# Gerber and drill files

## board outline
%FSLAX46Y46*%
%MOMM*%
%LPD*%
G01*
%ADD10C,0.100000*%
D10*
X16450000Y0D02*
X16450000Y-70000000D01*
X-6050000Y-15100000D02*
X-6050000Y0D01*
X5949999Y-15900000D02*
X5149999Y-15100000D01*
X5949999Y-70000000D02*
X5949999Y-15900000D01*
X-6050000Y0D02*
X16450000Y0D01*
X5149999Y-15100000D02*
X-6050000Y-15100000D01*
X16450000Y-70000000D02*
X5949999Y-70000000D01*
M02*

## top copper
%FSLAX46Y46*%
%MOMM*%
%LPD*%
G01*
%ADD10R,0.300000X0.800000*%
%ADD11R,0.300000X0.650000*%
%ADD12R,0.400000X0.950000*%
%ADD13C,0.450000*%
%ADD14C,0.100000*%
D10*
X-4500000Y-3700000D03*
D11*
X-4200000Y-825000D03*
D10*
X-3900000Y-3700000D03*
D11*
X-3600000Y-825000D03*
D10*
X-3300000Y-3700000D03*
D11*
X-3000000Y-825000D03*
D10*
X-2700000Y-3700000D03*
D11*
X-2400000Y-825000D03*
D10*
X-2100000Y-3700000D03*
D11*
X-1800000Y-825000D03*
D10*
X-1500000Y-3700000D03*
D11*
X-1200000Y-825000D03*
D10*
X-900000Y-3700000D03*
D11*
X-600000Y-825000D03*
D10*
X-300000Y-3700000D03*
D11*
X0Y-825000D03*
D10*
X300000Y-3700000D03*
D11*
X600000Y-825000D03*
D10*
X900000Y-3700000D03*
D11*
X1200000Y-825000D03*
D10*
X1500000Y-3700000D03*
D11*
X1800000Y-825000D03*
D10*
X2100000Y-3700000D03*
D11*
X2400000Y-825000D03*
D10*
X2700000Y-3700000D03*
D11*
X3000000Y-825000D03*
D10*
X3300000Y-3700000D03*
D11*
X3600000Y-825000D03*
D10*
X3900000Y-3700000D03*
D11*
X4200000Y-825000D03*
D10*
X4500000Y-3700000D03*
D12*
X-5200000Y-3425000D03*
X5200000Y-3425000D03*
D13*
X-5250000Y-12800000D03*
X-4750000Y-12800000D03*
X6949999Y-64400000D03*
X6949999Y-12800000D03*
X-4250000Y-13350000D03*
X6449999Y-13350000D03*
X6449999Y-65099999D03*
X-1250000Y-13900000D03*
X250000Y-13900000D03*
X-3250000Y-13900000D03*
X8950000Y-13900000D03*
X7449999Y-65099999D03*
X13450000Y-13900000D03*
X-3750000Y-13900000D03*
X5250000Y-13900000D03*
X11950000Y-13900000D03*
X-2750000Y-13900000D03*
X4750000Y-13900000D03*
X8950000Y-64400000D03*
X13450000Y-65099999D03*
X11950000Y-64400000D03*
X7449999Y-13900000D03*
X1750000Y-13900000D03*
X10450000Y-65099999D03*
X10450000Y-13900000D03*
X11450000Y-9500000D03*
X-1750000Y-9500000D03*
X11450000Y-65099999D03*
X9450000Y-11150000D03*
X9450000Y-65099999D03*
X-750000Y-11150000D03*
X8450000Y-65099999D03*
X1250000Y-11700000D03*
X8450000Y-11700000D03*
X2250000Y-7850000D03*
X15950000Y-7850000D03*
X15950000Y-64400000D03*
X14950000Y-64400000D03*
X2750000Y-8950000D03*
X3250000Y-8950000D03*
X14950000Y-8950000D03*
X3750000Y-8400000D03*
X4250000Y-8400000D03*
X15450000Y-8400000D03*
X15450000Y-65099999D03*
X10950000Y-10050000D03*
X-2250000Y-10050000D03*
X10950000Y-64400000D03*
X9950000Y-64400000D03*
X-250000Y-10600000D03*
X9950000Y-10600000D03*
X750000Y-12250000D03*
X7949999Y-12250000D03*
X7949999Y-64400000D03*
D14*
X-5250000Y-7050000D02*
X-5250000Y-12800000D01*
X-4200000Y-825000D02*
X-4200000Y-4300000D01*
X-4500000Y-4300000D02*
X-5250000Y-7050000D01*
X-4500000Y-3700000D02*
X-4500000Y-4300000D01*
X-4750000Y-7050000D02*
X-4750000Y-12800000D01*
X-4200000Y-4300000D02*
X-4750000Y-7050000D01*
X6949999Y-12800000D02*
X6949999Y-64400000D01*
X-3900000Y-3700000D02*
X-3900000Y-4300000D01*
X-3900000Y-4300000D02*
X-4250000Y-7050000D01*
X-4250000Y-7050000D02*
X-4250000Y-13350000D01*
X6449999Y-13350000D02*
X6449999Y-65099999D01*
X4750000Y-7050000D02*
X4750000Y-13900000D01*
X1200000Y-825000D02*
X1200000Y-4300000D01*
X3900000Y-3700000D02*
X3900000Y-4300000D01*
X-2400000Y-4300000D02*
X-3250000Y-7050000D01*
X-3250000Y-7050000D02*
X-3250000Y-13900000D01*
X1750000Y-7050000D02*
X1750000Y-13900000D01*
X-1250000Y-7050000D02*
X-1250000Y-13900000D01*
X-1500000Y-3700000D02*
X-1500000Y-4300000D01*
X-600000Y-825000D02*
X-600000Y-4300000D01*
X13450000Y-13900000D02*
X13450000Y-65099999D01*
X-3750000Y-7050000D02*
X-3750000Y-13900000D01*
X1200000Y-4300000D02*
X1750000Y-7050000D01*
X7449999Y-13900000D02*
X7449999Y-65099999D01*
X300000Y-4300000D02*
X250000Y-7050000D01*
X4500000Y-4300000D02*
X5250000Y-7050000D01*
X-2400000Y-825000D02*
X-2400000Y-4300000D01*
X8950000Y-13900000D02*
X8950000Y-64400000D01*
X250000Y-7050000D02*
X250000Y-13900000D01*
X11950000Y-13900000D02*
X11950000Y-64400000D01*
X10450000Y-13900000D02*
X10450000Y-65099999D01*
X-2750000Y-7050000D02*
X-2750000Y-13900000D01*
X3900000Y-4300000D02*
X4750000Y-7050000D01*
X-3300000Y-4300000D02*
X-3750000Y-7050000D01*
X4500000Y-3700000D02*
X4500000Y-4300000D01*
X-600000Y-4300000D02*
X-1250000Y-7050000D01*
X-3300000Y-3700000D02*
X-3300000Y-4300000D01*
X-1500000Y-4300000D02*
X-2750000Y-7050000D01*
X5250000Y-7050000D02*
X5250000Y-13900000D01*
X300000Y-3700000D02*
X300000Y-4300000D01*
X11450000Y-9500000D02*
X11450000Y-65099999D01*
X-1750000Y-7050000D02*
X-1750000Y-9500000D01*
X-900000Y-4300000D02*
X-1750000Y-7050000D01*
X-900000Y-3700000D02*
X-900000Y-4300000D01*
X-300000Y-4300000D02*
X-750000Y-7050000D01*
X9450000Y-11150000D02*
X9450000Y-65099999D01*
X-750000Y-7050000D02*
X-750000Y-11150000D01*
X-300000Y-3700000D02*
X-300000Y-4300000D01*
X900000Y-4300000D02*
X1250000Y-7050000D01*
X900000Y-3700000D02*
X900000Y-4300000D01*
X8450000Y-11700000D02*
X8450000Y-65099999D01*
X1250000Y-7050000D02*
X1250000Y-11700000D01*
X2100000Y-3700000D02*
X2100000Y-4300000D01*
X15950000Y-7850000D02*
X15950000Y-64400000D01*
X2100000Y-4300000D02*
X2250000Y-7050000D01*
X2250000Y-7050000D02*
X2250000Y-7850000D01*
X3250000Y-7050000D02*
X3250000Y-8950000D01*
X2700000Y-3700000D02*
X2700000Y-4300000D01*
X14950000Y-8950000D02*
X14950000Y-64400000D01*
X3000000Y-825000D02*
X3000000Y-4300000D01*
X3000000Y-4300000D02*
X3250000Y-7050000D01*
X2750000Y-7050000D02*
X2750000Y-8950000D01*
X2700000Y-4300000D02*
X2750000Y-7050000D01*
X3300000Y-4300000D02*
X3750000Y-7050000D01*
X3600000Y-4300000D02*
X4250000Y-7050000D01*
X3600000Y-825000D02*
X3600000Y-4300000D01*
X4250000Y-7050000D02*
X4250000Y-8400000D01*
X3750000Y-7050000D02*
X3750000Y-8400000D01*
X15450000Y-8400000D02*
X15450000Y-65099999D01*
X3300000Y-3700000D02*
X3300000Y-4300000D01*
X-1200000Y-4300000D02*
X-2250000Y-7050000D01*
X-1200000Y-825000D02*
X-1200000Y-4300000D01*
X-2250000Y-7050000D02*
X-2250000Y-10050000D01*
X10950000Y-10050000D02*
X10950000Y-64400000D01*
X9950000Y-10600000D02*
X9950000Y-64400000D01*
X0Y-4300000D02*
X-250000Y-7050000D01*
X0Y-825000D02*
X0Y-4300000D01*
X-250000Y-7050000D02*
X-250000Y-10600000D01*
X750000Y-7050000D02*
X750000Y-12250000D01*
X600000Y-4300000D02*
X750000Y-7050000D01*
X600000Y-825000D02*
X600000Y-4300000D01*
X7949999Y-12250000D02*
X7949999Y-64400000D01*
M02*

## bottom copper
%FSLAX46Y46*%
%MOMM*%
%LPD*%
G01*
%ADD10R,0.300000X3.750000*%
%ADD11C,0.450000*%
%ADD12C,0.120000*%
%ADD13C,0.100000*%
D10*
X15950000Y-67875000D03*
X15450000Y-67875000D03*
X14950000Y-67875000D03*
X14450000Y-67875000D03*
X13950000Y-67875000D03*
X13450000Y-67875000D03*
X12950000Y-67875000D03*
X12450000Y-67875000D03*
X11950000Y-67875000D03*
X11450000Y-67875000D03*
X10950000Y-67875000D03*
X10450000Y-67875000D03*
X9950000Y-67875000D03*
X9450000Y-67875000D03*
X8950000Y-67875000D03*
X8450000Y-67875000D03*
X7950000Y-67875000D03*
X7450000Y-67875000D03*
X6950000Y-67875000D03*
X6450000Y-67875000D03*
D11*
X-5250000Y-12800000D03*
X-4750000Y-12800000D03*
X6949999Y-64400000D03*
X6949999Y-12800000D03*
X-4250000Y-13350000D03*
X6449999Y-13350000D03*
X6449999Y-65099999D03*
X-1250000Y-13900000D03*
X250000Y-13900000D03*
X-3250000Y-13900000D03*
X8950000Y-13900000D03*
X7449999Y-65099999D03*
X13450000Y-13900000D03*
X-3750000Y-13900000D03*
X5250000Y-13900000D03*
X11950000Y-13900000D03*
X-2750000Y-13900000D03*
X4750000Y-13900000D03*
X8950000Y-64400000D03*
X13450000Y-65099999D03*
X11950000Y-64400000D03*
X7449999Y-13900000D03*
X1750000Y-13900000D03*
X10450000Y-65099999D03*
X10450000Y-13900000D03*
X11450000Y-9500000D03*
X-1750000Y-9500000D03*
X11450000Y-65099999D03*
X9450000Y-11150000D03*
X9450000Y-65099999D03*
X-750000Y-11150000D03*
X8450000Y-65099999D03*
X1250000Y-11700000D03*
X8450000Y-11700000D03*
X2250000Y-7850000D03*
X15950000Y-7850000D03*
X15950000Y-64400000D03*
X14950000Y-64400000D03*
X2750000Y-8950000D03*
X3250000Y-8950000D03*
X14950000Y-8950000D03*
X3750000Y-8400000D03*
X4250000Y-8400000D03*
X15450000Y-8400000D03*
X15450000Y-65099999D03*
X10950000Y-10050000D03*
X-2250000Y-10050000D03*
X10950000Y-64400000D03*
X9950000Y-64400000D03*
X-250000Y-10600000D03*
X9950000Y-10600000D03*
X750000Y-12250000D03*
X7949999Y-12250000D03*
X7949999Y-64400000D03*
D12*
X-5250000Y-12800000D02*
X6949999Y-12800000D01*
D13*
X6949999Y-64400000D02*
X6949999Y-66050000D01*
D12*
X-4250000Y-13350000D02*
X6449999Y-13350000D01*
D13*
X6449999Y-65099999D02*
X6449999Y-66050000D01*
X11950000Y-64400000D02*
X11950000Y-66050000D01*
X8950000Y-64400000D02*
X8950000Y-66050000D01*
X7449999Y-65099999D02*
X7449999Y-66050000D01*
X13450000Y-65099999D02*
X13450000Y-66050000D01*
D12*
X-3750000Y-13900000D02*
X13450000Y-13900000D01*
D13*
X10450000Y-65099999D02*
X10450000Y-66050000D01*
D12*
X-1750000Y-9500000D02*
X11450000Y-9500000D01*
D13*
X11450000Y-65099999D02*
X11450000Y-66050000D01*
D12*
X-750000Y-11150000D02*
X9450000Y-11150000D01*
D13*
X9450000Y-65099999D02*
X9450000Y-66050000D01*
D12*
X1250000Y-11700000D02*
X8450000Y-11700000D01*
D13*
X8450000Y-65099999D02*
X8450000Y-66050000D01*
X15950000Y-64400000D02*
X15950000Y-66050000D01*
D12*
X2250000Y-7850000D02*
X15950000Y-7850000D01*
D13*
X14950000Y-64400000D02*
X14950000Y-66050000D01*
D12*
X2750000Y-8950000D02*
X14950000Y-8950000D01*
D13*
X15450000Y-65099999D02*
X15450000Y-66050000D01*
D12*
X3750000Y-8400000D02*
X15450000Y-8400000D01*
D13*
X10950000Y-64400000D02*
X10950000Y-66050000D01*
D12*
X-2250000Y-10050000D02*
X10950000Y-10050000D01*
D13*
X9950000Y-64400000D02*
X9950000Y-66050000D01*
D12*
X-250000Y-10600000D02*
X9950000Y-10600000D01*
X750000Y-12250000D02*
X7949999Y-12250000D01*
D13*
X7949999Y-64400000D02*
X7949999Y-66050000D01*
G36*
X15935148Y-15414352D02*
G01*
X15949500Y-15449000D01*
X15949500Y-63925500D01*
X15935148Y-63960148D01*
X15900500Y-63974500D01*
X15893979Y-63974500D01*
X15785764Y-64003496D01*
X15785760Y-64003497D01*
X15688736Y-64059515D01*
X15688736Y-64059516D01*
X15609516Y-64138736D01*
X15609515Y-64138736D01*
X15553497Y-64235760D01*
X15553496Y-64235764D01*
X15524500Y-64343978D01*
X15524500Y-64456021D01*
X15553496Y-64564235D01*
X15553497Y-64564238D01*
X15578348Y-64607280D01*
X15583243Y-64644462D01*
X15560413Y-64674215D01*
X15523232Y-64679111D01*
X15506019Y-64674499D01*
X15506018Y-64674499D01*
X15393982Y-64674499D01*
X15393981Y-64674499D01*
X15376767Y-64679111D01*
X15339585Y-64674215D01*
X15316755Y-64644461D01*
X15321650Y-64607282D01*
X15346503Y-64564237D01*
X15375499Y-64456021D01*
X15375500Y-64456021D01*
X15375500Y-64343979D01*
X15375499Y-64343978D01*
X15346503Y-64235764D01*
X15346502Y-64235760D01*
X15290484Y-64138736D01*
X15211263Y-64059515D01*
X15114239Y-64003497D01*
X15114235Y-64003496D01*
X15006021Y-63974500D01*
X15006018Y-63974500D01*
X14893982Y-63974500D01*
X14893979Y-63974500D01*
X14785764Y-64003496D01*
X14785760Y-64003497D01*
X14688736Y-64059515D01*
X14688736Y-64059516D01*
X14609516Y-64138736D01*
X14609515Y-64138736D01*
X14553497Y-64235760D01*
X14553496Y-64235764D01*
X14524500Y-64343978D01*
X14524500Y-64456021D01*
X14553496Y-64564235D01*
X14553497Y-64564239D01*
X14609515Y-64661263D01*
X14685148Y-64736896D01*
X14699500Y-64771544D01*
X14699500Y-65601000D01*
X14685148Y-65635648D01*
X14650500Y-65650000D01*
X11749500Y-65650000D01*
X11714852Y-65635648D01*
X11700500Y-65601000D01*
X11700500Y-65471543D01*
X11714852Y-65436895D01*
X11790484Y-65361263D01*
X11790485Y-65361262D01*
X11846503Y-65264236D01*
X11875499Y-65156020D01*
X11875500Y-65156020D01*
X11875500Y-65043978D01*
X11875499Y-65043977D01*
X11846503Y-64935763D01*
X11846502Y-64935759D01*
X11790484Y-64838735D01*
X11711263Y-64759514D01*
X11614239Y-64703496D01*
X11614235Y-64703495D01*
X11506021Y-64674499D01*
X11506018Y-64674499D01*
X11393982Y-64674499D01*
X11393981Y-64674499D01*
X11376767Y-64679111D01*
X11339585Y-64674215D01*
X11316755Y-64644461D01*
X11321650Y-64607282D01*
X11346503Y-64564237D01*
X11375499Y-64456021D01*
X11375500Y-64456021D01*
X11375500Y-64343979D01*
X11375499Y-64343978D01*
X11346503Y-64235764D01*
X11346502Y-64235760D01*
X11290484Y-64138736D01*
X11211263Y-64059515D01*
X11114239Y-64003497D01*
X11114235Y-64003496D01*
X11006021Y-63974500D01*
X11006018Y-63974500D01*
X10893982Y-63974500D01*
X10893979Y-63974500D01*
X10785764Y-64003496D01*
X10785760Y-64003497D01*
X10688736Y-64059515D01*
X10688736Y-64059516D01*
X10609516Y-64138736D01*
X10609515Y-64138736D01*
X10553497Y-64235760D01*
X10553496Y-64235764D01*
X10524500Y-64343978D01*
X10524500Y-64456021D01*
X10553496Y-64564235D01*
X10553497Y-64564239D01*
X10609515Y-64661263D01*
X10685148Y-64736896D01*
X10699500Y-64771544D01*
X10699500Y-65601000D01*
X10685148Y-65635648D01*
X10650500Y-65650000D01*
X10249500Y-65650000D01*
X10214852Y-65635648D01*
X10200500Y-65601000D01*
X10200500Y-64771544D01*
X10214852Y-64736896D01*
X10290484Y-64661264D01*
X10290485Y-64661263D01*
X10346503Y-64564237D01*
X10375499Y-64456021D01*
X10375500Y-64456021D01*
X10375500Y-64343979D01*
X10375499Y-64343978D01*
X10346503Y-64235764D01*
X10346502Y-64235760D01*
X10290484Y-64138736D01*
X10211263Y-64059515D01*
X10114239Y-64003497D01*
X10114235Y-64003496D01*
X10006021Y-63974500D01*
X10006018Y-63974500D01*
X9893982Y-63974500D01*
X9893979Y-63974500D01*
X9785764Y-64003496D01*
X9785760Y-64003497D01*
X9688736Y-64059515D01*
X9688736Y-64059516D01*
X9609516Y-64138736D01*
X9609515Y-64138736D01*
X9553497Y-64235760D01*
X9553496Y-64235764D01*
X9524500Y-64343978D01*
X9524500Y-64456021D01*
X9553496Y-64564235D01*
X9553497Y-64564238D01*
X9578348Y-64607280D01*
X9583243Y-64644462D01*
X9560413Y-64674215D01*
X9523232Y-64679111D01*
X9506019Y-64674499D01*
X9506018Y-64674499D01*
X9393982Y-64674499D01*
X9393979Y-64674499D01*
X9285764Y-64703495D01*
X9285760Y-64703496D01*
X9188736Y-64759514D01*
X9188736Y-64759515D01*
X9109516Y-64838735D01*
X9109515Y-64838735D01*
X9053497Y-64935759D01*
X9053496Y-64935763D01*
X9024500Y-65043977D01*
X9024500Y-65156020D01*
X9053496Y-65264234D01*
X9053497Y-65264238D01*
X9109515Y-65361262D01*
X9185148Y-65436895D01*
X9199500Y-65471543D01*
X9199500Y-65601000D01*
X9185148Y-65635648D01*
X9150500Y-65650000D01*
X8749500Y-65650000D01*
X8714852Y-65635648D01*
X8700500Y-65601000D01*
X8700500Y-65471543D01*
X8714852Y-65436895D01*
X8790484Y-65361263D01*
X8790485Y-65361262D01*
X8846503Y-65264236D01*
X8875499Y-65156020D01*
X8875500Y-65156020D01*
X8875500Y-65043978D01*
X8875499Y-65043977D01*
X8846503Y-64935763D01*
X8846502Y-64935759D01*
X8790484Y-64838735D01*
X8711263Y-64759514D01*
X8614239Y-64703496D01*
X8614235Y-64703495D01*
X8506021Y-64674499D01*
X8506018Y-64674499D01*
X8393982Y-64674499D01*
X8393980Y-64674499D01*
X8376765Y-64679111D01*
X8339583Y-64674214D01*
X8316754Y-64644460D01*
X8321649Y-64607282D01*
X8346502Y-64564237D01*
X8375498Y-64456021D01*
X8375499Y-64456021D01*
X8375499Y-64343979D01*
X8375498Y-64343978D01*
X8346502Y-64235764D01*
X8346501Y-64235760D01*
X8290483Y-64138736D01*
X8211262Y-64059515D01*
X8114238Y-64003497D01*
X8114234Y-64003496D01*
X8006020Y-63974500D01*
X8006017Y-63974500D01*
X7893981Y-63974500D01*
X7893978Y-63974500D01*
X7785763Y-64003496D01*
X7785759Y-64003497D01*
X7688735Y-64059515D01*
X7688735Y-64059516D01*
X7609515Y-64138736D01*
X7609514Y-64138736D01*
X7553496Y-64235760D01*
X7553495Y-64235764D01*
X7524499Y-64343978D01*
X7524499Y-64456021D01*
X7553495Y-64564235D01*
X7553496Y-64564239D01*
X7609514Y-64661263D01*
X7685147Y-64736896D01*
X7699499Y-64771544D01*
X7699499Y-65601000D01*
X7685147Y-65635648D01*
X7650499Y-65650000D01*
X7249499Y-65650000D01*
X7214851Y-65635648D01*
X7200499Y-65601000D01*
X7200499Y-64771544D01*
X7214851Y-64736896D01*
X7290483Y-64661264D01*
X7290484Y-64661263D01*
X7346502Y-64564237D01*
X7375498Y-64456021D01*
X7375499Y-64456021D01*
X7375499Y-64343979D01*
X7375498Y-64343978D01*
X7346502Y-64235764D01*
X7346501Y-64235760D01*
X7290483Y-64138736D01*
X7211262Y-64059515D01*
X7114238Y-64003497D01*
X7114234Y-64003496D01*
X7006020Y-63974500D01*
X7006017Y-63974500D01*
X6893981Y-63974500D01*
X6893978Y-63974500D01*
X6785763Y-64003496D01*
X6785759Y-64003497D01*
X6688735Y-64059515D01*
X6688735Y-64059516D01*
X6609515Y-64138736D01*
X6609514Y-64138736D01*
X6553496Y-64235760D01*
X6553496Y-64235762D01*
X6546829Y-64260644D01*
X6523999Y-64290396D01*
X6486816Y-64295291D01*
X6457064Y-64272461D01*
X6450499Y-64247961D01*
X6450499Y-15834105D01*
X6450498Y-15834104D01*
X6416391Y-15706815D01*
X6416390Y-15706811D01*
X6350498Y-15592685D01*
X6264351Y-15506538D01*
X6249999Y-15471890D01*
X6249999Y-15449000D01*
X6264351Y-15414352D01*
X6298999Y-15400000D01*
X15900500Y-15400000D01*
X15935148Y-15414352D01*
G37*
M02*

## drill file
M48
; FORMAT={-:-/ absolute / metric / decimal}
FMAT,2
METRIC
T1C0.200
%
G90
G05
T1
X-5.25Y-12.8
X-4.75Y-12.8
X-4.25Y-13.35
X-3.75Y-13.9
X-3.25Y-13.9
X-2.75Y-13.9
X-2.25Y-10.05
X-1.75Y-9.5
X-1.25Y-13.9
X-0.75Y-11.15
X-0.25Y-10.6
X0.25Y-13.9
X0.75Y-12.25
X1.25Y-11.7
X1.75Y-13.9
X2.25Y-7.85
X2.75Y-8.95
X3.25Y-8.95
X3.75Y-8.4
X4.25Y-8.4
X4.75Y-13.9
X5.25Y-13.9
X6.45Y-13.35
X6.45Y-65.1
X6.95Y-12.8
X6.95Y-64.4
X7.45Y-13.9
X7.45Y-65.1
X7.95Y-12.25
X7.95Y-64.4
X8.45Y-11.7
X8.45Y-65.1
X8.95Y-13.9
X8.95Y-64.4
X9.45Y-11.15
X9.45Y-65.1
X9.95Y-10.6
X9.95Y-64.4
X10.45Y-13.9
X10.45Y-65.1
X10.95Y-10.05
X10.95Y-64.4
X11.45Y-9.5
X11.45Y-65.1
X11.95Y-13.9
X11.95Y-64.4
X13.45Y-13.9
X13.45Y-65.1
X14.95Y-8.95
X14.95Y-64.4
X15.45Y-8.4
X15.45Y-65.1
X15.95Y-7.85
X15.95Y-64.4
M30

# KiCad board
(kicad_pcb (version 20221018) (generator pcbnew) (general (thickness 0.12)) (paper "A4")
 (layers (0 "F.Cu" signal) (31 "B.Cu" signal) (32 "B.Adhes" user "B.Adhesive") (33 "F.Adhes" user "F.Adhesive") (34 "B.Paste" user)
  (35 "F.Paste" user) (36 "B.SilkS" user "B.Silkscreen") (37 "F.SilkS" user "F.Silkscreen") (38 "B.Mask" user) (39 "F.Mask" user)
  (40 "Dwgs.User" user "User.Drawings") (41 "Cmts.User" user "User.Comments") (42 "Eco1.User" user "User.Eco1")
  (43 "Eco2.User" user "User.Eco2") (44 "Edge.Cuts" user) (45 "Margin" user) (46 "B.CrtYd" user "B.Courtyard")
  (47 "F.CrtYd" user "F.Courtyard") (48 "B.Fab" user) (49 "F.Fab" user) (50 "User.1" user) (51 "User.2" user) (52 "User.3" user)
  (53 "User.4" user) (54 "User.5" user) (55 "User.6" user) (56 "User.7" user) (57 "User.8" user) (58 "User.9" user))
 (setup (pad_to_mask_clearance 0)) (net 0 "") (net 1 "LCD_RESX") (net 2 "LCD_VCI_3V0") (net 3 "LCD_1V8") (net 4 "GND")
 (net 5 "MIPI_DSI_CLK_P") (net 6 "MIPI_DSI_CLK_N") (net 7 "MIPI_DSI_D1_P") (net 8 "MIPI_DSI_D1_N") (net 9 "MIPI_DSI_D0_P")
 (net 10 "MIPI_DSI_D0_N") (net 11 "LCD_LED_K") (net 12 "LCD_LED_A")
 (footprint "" (layer "F.Cu") (at 11.2 67.875)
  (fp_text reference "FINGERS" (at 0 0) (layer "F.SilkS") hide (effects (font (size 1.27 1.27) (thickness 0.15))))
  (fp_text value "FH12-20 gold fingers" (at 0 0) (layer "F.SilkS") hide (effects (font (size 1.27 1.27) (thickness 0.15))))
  (pad "1" smd rect (at 4.75 0) (size 0.3 3.75) (layers "B.Cu" "B.Mask") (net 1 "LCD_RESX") (thermal_bridge_angle 45))
  (pad "2" smd rect (at 4.25 0) (size 0.3 3.75) (layers "B.Cu" "B.Mask") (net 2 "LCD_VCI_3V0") (thermal_bridge_angle 45))
  (pad "3" smd rect (at 3.75 0) (size 0.3 3.75) (layers "B.Cu" "B.Mask") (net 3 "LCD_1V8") (thermal_bridge_angle 45))
  (pad "4" smd rect (at 3.25 0) (size 0.3 3.75) (layers "B.Cu" "B.Mask") (thermal_bridge_angle 45))
  (pad "5" smd rect (at 2.75 0) (size 0.3 3.75) (layers "B.Cu" "B.Mask") (thermal_bridge_angle 45))
  (pad "6" smd rect (at 2.25 0) (size 0.3 3.75) (layers "B.Cu" "B.Mask") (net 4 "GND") (thermal_bridge_angle 45))
  (pad "7" smd rect (at 1.75 0) (size 0.3 3.75) (layers "B.Cu" "B.Mask") (thermal_bridge_angle 45))
  (pad "8" smd rect (at 1.25 0) (size 0.3 3.75) (layers "B.Cu" "B.Mask") (thermal_bridge_angle 45))
  (pad "9" smd rect (at 0.75 0) (size 0.3 3.75) (layers "B.Cu" "B.Mask") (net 4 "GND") (thermal_bridge_angle 45))
  (pad "10" smd rect (at 0.25 0) (size 0.3 3.75) (layers "B.Cu" "B.Mask") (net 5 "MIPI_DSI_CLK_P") (thermal_bridge_angle 45))
  (pad "11" smd rect (at -0.25 0) (size 0.3 3.75) (layers "B.Cu" "B.Mask") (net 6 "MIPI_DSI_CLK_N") (thermal_bridge_angle 45))
  (pad "12" smd rect (at -0.75 0) (size 0.3 3.75) (layers "B.Cu" "B.Mask") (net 4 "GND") (thermal_bridge_angle 45))
  (pad "13" smd rect (at -1.25 0) (size 0.3 3.75) (layers "B.Cu" "B.Mask") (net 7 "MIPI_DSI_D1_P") (thermal_bridge_angle 45))
  (pad "14" smd rect (at -1.75 0) (size 0.3 3.75) (layers "B.Cu" "B.Mask") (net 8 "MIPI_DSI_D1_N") (thermal_bridge_angle 45))
  (pad "15" smd rect (at -2.25 0) (size 0.3 3.75) (layers "B.Cu" "B.Mask") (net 4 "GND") (thermal_bridge_angle 45))
  (pad "16" smd rect (at -2.75 0) (size 0.3 3.75) (layers "B.Cu" "B.Mask") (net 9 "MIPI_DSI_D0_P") (thermal_bridge_angle 45))
  (pad "17" smd rect (at -3.25 0) (size 0.3 3.75) (layers "B.Cu" "B.Mask") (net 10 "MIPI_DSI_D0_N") (thermal_bridge_angle 45))
  (pad "18" smd rect (at -3.75 0) (size 0.3 3.75) (layers "B.Cu" "B.Mask") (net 4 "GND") (thermal_bridge_angle 45))
  (pad "19" smd rect (at -4.25 0) (size 0.3 3.75) (layers "B.Cu" "B.Mask") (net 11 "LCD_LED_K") (thermal_bridge_angle 45))
  (pad "20" smd rect (at -4.75 0) (size 0.3 3.75) (layers "B.Cu" "B.Mask") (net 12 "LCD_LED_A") (thermal_bridge_angle 45)))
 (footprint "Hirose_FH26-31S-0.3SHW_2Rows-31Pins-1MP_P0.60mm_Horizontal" (layer "F.Cu") (at 0 2.3 90)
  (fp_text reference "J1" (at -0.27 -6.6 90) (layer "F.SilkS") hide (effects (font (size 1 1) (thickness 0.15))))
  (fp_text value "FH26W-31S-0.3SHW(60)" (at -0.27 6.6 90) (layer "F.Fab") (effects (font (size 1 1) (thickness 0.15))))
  (pad "1" smd rect (at -1.4 -4.5 90) (size 0.8 0.3) (layers "F.Cu" "F.Paste" "F.Mask") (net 11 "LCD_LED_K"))
  (pad "2" smd rect (at 1.475 -4.2 90) (size 0.65 0.3) (layers "F.Cu" "F.Paste" "F.Mask") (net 11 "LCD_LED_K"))
  (pad "3" smd rect (at -1.4 -3.9 90) (size 0.8 0.3) (layers "F.Cu" "F.Paste" "F.Mask") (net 12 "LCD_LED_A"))
  (pad "4" smd rect (at 1.475 -3.6 90) (size 0.65 0.3) (layers "F.Cu" "F.Paste" "F.Mask"))
  (pad "5" smd rect (at -1.4 -3.3 90) (size 0.8 0.3) (layers "F.Cu" "F.Paste" "F.Mask") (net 4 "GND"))
  (pad "6" smd rect (at 1.475 -3 90) (size 0.65 0.3) (layers "F.Cu" "F.Paste" "F.Mask"))
  (pad "7" smd rect (at -1.4 -2.7 90) (size 0.8 0.3) (layers "F.Cu" "F.Paste" "F.Mask"))
  (pad "8" smd rect (at 1.475 -2.4 90) (size 0.65 0.3) (layers "F.Cu" "F.Paste" "F.Mask") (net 4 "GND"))
  (pad "9" smd rect (at -1.4 -2.1 90) (size 0.8 0.3) (layers "F.Cu" "F.Paste" "F.Mask"))
  (pad "10" smd rect (at 1.475 -1.8 90) (size 0.65 0.3) (layers "F.Cu" "F.Paste" "F.Mask"))
  (pad "11" smd rect (at -1.4 -1.5 90) (size 0.8 0.3) (layers "F.Cu" "F.Paste" "F.Mask") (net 4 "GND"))
  (pad "12" smd rect (at 1.475 -1.2 90) (size 0.65 0.3) (layers "F.Cu" "F.Paste" "F.Mask") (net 6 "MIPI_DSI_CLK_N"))
  (pad "13" smd rect (at -1.4 -0.9 90) (size 0.8 0.3) (layers "F.Cu" "F.Paste" "F.Mask") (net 5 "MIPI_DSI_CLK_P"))
  (pad "14" smd rect (at 1.475 -0.6 90) (size 0.65 0.3) (layers "F.Cu" "F.Paste" "F.Mask") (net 4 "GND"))
  (pad "15" smd rect (at -1.4 -0.3 90) (size 0.8 0.3) (layers "F.Cu" "F.Paste" "F.Mask") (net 8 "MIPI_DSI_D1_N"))
  (pad "16" smd rect (at 1.475 0 90) (size 0.65 0.3) (layers "F.Cu" "F.Paste" "F.Mask") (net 7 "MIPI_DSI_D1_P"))
  (pad "17" smd rect (at -1.4 0.3 90) (size 0.8 0.3) (layers "F.Cu" "F.Paste" "F.Mask") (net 4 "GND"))
  (pad "18" smd rect (at 1.475 0.6 90) (size 0.65 0.3) (layers "F.Cu" "F.Paste" "F.Mask") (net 10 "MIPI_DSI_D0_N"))
  (pad "19" smd rect (at -1.4 0.9 90) (size 0.8 0.3) (layers "F.Cu" "F.Paste" "F.Mask") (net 9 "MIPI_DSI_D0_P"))
  (pad "20" smd rect (at 1.475 1.2 90) (size 0.65 0.3) (layers "F.Cu" "F.Paste" "F.Mask") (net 4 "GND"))
  (pad "21" smd rect (at -1.4 1.5 90) (size 0.8 0.3) (layers "F.Cu" "F.Paste" "F.Mask"))
  (pad "22" smd rect (at 1.475 1.8 90) (size 0.65 0.3) (layers "F.Cu" "F.Paste" "F.Mask"))
  (pad "23" smd rect (at -1.4 2.1 90) (size 0.8 0.3) (layers "F.Cu" "F.Paste" "F.Mask") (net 1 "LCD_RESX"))
  (pad "24" smd rect (at 1.475 2.4 90) (size 0.65 0.3) (layers "F.Cu" "F.Paste" "F.Mask"))
  (pad "25" smd rect (at -1.4 2.7 90) (size 0.8 0.3) (layers "F.Cu" "F.Paste" "F.Mask") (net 3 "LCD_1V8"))
  (pad "26" smd rect (at 1.475 3 90) (size 0.65 0.3) (layers "F.Cu" "F.Paste" "F.Mask") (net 3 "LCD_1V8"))
  (pad "27" smd rect (at -1.4 3.3 90) (size 0.8 0.3) (layers "F.Cu" "F.Paste" "F.Mask") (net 2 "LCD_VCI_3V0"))
  (pad "28" smd rect (at 1.475 3.6 90) (size 0.65 0.3) (layers "F.Cu" "F.Paste" "F.Mask") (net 2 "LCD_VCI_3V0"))
  (pad "29" smd rect (at -1.4 3.9 90) (size 0.8 0.3) (layers "F.Cu" "F.Paste" "F.Mask") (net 4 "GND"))
  (pad "30" smd rect (at 1.475 4.2 90) (size 0.65 0.3) (layers "F.Cu" "F.Paste" "F.Mask"))
  (pad "31" smd rect (at -1.4 4.5 90) (size 0.8 0.3) (layers "F.Cu" "F.Paste" "F.Mask") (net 4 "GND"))
  (pad "MP" smd rect (at -1.125 -5.2 90) (size 0.95 0.4) (layers "F.Cu" "F.Paste" "F.Mask"))
  (pad "MP" smd rect (at -1.125 5.2 90) (size 0.95 0.4) (layers "F.Cu" "F.Paste" "F.Mask")))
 (gr_line (start 16.45 0) (end 16.45 70) (stroke (width 0.1) (type default)) (layer "Edge.Cuts"))
 (gr_line (start -6.05 15.1) (end -6.05 0) (stroke (width 0.1) (type default)) (layer "Edge.Cuts"))
 (gr_line (start 5.949999 15.9) (end 5.149999 15.1) (stroke (width 0.1) (type default)) (layer "Edge.Cuts"))
 (gr_line (start 5.949999 70) (end 5.949999 15.9) (stroke (width 0.1) (type default)) (layer "Edge.Cuts"))
 (gr_line (start -6.05 0) (end 16.45 0) (stroke (width 0.1) (type default)) (layer "Edge.Cuts"))
 (gr_line (start 5.149999 15.1) (end -6.05 15.1) (stroke (width 0.1) (type default)) (layer "Edge.Cuts"))
 (gr_line (start 16.45 70) (end 5.949999 70) (stroke (width 0.1) (type default)) (layer "Edge.Cuts"))
 (segment (start -5.25 7.05) (end -5.25 12.8) (width 0.1) (layer "F.Cu") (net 11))
 (segment (start -4.2 0.825) (end -4.2 4.3) (width 0.1) (layer "F.Cu") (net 11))
 (segment (start -4.5 4.3) (end -5.25 7.05) (width 0.1) (layer "F.Cu") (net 11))
 (segment (start -4.5 3.7) (end -4.5 4.3) (width 0.1) (layer "F.Cu") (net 11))
 (segment (start -4.75 7.05) (end -4.75 12.8) (width 0.1) (layer "F.Cu") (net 11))
 (segment (start -4.2 4.3) (end -4.75 7.05) (width 0.1) (layer "F.Cu") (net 11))
 (segment (start 6.949999 12.8) (end 6.949999 64.4) (width 0.1) (layer "F.Cu") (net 11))
 (via (at -5.25 12.8) (size 0.45) (drill 0.2) (layers "F.Cu" "B.Cu") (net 11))
 (via (at -4.75 12.8) (size 0.45) (drill 0.2) (layers "F.Cu" "B.Cu") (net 11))
 (via (at 6.949999 64.4) (size 0.45) (drill 0.2) (layers "F.Cu" "B.Cu") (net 11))
 (via (at 6.949999 12.8) (size 0.45) (drill 0.2) (layers "F.Cu" "B.Cu") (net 11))
 (segment (start -5.25 12.8) (end 6.949999 12.8) (width 0.12) (layer "B.Cu") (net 11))
 (segment (start 6.949999 64.4) (end 6.949999 66.05) (width 0.1) (layer "B.Cu") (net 11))
 (segment (start -3.9 3.7) (end -3.9 4.3) (width 0.1) (layer "F.Cu") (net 12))
 (segment (start -3.9 4.3) (end -4.25 7.05) (width 0.1) (layer "F.Cu") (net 12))
 (segment (start -4.25 7.05) (end -4.25 13.35) (width 0.1) (layer "F.Cu") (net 12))
 (segment (start 6.449999 13.35) (end 6.449999 65.099999) (width 0.1) (layer "F.Cu") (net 12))
 (via (at -4.25 13.35) (size 0.45) (drill 0.2) (layers "F.Cu" "B.Cu") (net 12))
 (via (at 6.449999 13.35) (size 0.45) (drill 0.2) (layers "F.Cu" "B.Cu") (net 12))
 (via (at 6.449999 65.099999) (size 0.45) (drill 0.2) (layers "F.Cu" "B.Cu") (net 12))
 (segment (start -4.25 13.35) (end 6.449999 13.35) (width 0.12) (layer "B.Cu") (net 12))
 (segment (start 6.449999 65.099999) (end 6.449999 66.05) (width 0.1) (layer "B.Cu") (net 12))
 (segment (start 4.75 7.05) (end 4.75 13.9) (width 0.1) (layer "F.Cu") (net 4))
 (segment (start 1.2 0.825) (end 1.2 4.3) (width 0.1) (layer "F.Cu") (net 4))
 (segment (start 3.9 3.7) (end 3.9 4.3) (width 0.1) (layer "F.Cu") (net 4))
 (segment (start -2.4 4.3) (end -3.25 7.05) (width 0.1) (layer "F.Cu") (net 4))
 (segment (start -3.25 7.05) (end -3.25 13.9) (width 0.1) (layer "F.Cu") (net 4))
 (segment (start 1.75 7.05) (end 1.75 13.9) (width 0.1) (layer "F.Cu") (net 4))
 (segment (start -1.25 7.05) (end -1.25 13.9) (width 0.1) (layer "F.Cu") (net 4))
 (segment (start -1.5 3.7) (end -1.5 4.3) (width 0.1) (layer "F.Cu") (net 4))
 (segment (start -0.6 0.825) (end -0.6 4.3) (width 0.1) (layer "F.Cu") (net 4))
 (segment (start 13.45 13.9) (end 13.45 65.099999) (width 0.1) (layer "F.Cu") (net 4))
 (segment (start -3.75 7.05) (end -3.75 13.9) (width 0.1) (layer "F.Cu") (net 4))
 (segment (start 1.2 4.3) (end 1.75 7.05) (width 0.1) (layer "F.Cu") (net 4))
 (segment (start 7.449999 13.9) (end 7.449999 65.099999) (width 0.1) (layer "F.Cu") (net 4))
 (segment (start 0.3 4.3) (end 0.25 7.05) (width 0.1) (layer "F.Cu") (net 4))
 (segment (start 4.5 4.3) (end 5.25 7.05) (width 0.1) (layer "F.Cu") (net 4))
 (segment (start -2.4 0.825) (end -2.4 4.3) (width 0.1) (layer "F.Cu") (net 4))
 (segment (start 8.95 13.9) (end 8.95 64.4) (width 0.1) (layer "F.Cu") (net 4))
 (segment (start 0.25 7.05) (end 0.25 13.9) (width 0.1) (layer "F.Cu") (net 4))
 (segment (start 11.95 13.9) (end 11.95 64.4) (width 0.1) (layer "F.Cu") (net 4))
 (segment (start 10.45 13.9) (end 10.45 65.099999) (width 0.1) (layer "F.Cu") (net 4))
 (segment (start -2.75 7.05) (end -2.75 13.9) (width 0.1) (layer "F.Cu") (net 4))
 (segment (start 3.9 4.3) (end 4.75 7.05) (width 0.1) (layer "F.Cu") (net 4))
 (segment (start -3.3 4.3) (end -3.75 7.05) (width 0.1) (layer "F.Cu") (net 4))
 (segment (start 4.5 3.7) (end 4.5 4.3) (width 0.1) (layer "F.Cu") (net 4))
 (segment (start -0.6 4.3) (end -1.25 7.05) (width 0.1) (layer "F.Cu") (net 4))
 (segment (start -3.3 3.7) (end -3.3 4.3) (width 0.1) (layer "F.Cu") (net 4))
 (segment (start -1.5 4.3) (end -2.75 7.05) (width 0.1) (layer "F.Cu") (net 4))
 (segment (start 5.25 7.05) (end 5.25 13.9) (width 0.1) (layer "F.Cu") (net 4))
 (segment (start 0.3 3.7) (end 0.3 4.3) (width 0.1) (layer "F.Cu") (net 4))
 (via (at -1.25 13.9) (size 0.45) (drill 0.2) (layers "F.Cu" "B.Cu") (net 4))
 (via (at 0.25 13.9) (size 0.45) (drill 0.2) (layers "F.Cu" "B.Cu") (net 4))
 (via (at -3.25 13.9) (size 0.45) (drill 0.2) (layers "F.Cu" "B.Cu") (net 4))
 (via (at 8.95 13.9) (size 0.45) (drill 0.2) (layers "F.Cu" "B.Cu") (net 4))
 (via (at 7.449999 65.099999) (size 0.45) (drill 0.2) (layers "F.Cu" "B.Cu") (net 4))
 (via (at 13.45 13.9) (size 0.45) (drill 0.2) (layers "F.Cu" "B.Cu") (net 4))
 (via (at -3.75 13.9) (size 0.45) (drill 0.2) (layers "F.Cu" "B.Cu") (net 4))
 (via (at 5.25 13.9) (size 0.45) (drill 0.2) (layers "F.Cu" "B.Cu") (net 4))
 (via (at 11.95 13.9) (size 0.45) (drill 0.2) (layers "F.Cu" "B.Cu") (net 4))
 (via (at -2.75 13.9) (size 0.45) (drill 0.2) (layers "F.Cu" "B.Cu") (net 4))
 (via (at 4.75 13.9) (size 0.45) (drill 0.2) (layers "F.Cu" "B.Cu") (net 4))
 (via (at 8.95 64.4) (size 0.45) (drill 0.2) (layers "F.Cu" "B.Cu") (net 4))
 (via (at 13.45 65.099999) (size 0.45) (drill 0.2) (layers "F.Cu" "B.Cu") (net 4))
 (via (at 11.95 64.4) (size 0.45) (drill 0.2) (layers "F.Cu" "B.Cu") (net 4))
 (via (at 7.449999 13.9) (size 0.45) (drill 0.2) (layers "F.Cu" "B.Cu") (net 4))
 (via (at 1.75 13.9) (size 0.45) (drill 0.2) (layers "F.Cu" "B.Cu") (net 4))
 (via (at 10.45 65.099999) (size 0.45) (drill 0.2) (layers "F.Cu" "B.Cu") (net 4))
 (via (at 10.45 13.9) (size 0.45) (drill 0.2) (layers "F.Cu" "B.Cu") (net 4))
 (segment (start 11.95 64.4) (end 11.95 66.05) (width 0.1) (layer "B.Cu") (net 4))
 (segment (start 8.95 64.4) (end 8.95 66.05) (width 0.1) (layer "B.Cu") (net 4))
 (segment (start 7.449999 65.099999) (end 7.449999 66.05) (width 0.1) (layer "B.Cu") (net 4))
 (segment (start 13.45 65.099999) (end 13.45 66.05) (width 0.1) (layer "B.Cu") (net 4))
 (segment (start -3.75 13.9) (end 13.45 13.9) (width 0.12) (layer "B.Cu") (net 4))
 (segment (start 10.45 65.099999) (end 10.45 66.05) (width 0.1) (layer "B.Cu") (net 4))
 (segment (start 11.45 9.5) (end 11.45 65.099999) (width 0.1) (layer "F.Cu") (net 5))
 (segment (start -1.75 7.05) (end -1.75 9.5) (width 0.1) (layer "F.Cu") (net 5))
 (segment (start -0.9 4.3) (end -1.75 7.05) (width 0.1) (layer "F.Cu") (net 5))
 (segment (start -0.9 3.7) (end -0.9 4.3) (width 0.1) (layer "F.Cu") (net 5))
 (via (at 11.45 9.5) (size 0.45) (drill 0.2) (layers "F.Cu" "B.Cu") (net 5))
 (via (at -1.75 9.5) (size 0.45) (drill 0.2) (layers "F.Cu" "B.Cu") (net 5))
 (via (at 11.45 65.099999) (size 0.45) (drill 0.2) (layers "F.Cu" "B.Cu") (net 5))
 (segment (start -1.75 9.5) (end 11.45 9.5) (width 0.12) (layer "B.Cu") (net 5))
 (segment (start 11.45 65.099999) (end 11.45 66.05) (width 0.1) (layer "B.Cu") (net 5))
 (segment (start -0.3 4.3) (end -0.75 7.05) (width 0.1) (layer "F.Cu") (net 8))
 (segment (start 9.45 11.15) (end 9.45 65.099999) (width 0.1) (layer "F.Cu") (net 8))
 (segment (start -0.75 7.05) (end -0.75 11.15) (width 0.1) (layer "F.Cu") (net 8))
 (segment (start -0.3 3.7) (end -0.3 4.3) (width 0.1) (layer "F.Cu") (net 8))
 (via (at 9.45 11.15) (size 0.45) (drill 0.2) (layers "F.Cu" "B.Cu") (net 8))
 (via (at 9.45 65.099999) (size 0.45) (drill 0.2) (layers "F.Cu" "B.Cu") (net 8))
 (via (at -0.75 11.15) (size 0.45) (drill 0.2) (layers "F.Cu" "B.Cu") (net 8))
 (segment (start -0.75 11.15) (end 9.45 11.15) (width 0.12) (layer "B.Cu") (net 8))
 (segment (start 9.45 65.099999) (end 9.45 66.05) (width 0.1) (layer "B.Cu") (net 8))
 (segment (start 0.9 4.3) (end 1.25 7.05) (width 0.1) (layer "F.Cu") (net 9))
 (segment (start 0.9 3.7) (end 0.9 4.3) (width 0.1) (layer "F.Cu") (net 9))
 (segment (start 8.45 11.7) (end 8.45 65.099999) (width 0.1) (layer "F.Cu") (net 9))
 (segment (start 1.25 7.05) (end 1.25 11.7) (width 0.1) (layer "F.Cu") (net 9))
 (via (at 8.45 65.099999) (size 0.45) (drill 0.2) (layers "F.Cu" "B.Cu") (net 9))
 (via (at 1.25 11.7) (size 0.45) (drill 0.2) (layers "F.Cu" "B.Cu") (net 9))
 (via (at 8.45 11.7) (size 0.45) (drill 0.2) (layers "F.Cu" "B.Cu") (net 9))
 (segment (start 1.25 11.7) (end 8.45 11.7) (width 0.12) (layer "B.Cu") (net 9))
 (segment (start 8.45 65.099999) (end 8.45 66.05) (width 0.1) (layer "B.Cu") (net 9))
 (segment (start 2.1 3.7) (end 2.1 4.3) (width 0.1) (layer "F.Cu") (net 1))
 (segment (start 15.95 7.85) (end 15.95 64.4) (width 0.1) (layer "F.Cu") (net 1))
 (segment (start 2.1 4.3) (end 2.25 7.05) (width 0.1) (layer "F.Cu") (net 1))
 (segment (start 2.25 7.05) (end 2.25 7.85) (width 0.1) (layer "F.Cu") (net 1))
 (via (at 2.25 7.85) (size 0.45) (drill 0.2) (layers "F.Cu" "B.Cu") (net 1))
 (via (at 15.95 7.85) (size 0.45) (drill 0.2) (layers "F.Cu" "B.Cu") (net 1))
 (via (at 15.95 64.4) (size 0.45) (drill 0.2) (layers "F.Cu" "B.Cu") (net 1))
 (segment (start 15.95 64.4) (end 15.95 66.05) (width 0.1) (layer "B.Cu") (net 1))
 (segment (start 2.25 7.85) (end 15.95 7.85) (width 0.12) (layer "B.Cu") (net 1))
 (segment (start 3.25 7.05) (end 3.25 8.95) (width 0.1) (layer "F.Cu") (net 3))
 (segment (start 2.7 3.7) (end 2.7 4.3) (width 0.1) (layer "F.Cu") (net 3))
 (segment (start 14.95 8.95) (end 14.95 64.4) (width 0.1) (layer "F.Cu") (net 3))
 (segment (start 3 0.825) (end 3 4.3) (width 0.1) (layer "F.Cu") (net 3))
 (segment (start 3 4.3) (end 3.25 7.05) (width 0.1) (layer "F.Cu") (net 3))
 (segment (start 2.75 7.05) (end 2.75 8.95) (width 0.1) (layer "F.Cu") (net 3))
 (segment (start 2.7 4.3) (end 2.75 7.05) (width 0.1) (layer "F.Cu") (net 3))
 (via (at 14.95 64.4) (size 0.45) (drill 0.2) (layers "F.Cu" "B.Cu") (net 3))
 (via (at 2.75 8.95) (size 0.45) (drill 0.2) (layers "F.Cu" "B.Cu") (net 3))
 (via (at 3.25 8.95) (size 0.45) (drill 0.2) (layers "F.Cu" "B.Cu") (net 3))
 (via (at 14.95 8.95) (size 0.45) (drill 0.2) (layers "F.Cu" "B.Cu") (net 3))
 (segment (start 14.95 64.4) (end 14.95 66.05) (width 0.1) (layer "B.Cu") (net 3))
 (segment (start 2.75 8.95) (end 14.95 8.95) (width 0.12) (layer "B.Cu") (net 3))
 (segment (start 3.3 4.3) (end 3.75 7.05) (width 0.1) (layer "F.Cu") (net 2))
 (segment (start 3.6 4.3) (end 4.25 7.05) (width 0.1) (layer "F.Cu") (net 2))
 (segment (start 3.6 0.825) (end 3.6 4.3) (width 0.1) (layer "F.Cu") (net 2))
 (segment (start 4.25 7.05) (end 4.25 8.4) (width 0.1) (layer "F.Cu") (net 2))
 (segment (start 3.75 7.05) (end 3.75 8.4) (width 0.1) (layer "F.Cu") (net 2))
 (segment (start 15.45 8.4) (end 15.45 65.099999) (width 0.1) (layer "F.Cu") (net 2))
 (segment (start 3.3 3.7) (end 3.3 4.3) (width 0.1) (layer "F.Cu") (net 2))
 (via (at 3.75 8.4) (size 0.45) (drill 0.2) (layers "F.Cu" "B.Cu") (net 2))
 (via (at 4.25 8.4) (size 0.45) (drill 0.2) (layers "F.Cu" "B.Cu") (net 2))
 (via (at 15.45 8.4) (size 0.45) (drill 0.2) (layers "F.Cu" "B.Cu") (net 2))
 (via (at 15.45 65.099999) (size 0.45) (drill 0.2) (layers "F.Cu" "B.Cu") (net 2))
 (segment (start 15.45 65.099999) (end 15.45 66.05) (width 0.1) (layer "B.Cu") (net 2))
 (segment (start 3.75 8.4) (end 15.45 8.4) (width 0.12) (layer "B.Cu") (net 2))
 (segment (start -1.2 4.3) (end -2.25 7.05) (width 0.1) (layer "F.Cu") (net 6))
 (segment (start -1.2 0.825) (end -1.2 4.3) (width 0.1) (layer "F.Cu") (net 6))
 (segment (start -2.25 7.05) (end -2.25 10.05) (width 0.1) (layer "F.Cu") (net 6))
 (segment (start 10.95 10.05) (end 10.95 64.4) (width 0.1) (layer "F.Cu") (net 6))
 (via (at 10.95 10.05) (size 0.45) (drill 0.2) (layers "F.Cu" "B.Cu") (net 6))
 (via (at -2.25 10.05) (size 0.45) (drill 0.2) (layers "F.Cu" "B.Cu") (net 6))
 (via (at 10.95 64.4) (size 0.45) (drill 0.2) (layers "F.Cu" "B.Cu") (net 6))
 (segment (start 10.95 64.4) (end 10.95 66.05) (width 0.1) (layer "B.Cu") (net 6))
 (segment (start -2.25 10.05) (end 10.95 10.05) (width 0.12) (layer "B.Cu") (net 6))
 (segment (start 9.95 10.6) (end 9.95 64.4) (width 0.1) (layer "F.Cu") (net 7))
 (segment (start 0 4.3) (end -0.25 7.05) (width 0.1) (layer "F.Cu") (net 7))
 (segment (start 0 0.825) (end 0 4.3) (width 0.1) (layer "F.Cu") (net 7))
 (segment (start -0.25 7.05) (end -0.25 10.6) (width 0.1) (layer "F.Cu") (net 7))
 (via (at 9.95 64.4) (size 0.45) (drill 0.2) (layers "F.Cu" "B.Cu") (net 7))
 (via (at -0.25 10.6) (size 0.45) (drill 0.2) (layers "F.Cu" "B.Cu") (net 7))
 (via (at 9.95 10.6) (size 0.45) (drill 0.2) (layers "F.Cu" "B.Cu") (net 7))
 (segment (start 9.95 64.4) (end 9.95 66.05) (width 0.1) (layer "B.Cu") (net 7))
 (segment (start -0.25 10.6) (end 9.95 10.6) (width 0.12) (layer "B.Cu") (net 7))
 (segment (start 0.75 7.05) (end 0.75 12.25) (width 0.1) (layer "F.Cu") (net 10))
 (segment (start 0.6 4.3) (end 0.75 7.05) (width 0.1) (layer "F.Cu") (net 10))
 (segment (start 0.6 0.825) (end 0.6 4.3) (width 0.1) (layer "F.Cu") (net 10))
 (segment (start 7.949999 12.25) (end 7.949999 64.4) (width 0.1) (layer "F.Cu") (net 10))
 (via (at 0.75 12.25) (size 0.45) (drill 0.2) (layers "F.Cu" "B.Cu") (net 10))
 (via (at 7.949999 12.25) (size 0.45) (drill 0.2) (layers "F.Cu" "B.Cu") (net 10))
 (via (at 7.949999 64.4) (size 0.45) (drill 0.2) (layers "F.Cu" "B.Cu") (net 10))
 (segment (start 0.75 12.25) (end 7.949999 12.25) (width 0.12) (layer "B.Cu") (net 10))
 (segment (start 7.949999 64.4) (end 7.949999 66.05) (width 0.1) (layer "B.Cu") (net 10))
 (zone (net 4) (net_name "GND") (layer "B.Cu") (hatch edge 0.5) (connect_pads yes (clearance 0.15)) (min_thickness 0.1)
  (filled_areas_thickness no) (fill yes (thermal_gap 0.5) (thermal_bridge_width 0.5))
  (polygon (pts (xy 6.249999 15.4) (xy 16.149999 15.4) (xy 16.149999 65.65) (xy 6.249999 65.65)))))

